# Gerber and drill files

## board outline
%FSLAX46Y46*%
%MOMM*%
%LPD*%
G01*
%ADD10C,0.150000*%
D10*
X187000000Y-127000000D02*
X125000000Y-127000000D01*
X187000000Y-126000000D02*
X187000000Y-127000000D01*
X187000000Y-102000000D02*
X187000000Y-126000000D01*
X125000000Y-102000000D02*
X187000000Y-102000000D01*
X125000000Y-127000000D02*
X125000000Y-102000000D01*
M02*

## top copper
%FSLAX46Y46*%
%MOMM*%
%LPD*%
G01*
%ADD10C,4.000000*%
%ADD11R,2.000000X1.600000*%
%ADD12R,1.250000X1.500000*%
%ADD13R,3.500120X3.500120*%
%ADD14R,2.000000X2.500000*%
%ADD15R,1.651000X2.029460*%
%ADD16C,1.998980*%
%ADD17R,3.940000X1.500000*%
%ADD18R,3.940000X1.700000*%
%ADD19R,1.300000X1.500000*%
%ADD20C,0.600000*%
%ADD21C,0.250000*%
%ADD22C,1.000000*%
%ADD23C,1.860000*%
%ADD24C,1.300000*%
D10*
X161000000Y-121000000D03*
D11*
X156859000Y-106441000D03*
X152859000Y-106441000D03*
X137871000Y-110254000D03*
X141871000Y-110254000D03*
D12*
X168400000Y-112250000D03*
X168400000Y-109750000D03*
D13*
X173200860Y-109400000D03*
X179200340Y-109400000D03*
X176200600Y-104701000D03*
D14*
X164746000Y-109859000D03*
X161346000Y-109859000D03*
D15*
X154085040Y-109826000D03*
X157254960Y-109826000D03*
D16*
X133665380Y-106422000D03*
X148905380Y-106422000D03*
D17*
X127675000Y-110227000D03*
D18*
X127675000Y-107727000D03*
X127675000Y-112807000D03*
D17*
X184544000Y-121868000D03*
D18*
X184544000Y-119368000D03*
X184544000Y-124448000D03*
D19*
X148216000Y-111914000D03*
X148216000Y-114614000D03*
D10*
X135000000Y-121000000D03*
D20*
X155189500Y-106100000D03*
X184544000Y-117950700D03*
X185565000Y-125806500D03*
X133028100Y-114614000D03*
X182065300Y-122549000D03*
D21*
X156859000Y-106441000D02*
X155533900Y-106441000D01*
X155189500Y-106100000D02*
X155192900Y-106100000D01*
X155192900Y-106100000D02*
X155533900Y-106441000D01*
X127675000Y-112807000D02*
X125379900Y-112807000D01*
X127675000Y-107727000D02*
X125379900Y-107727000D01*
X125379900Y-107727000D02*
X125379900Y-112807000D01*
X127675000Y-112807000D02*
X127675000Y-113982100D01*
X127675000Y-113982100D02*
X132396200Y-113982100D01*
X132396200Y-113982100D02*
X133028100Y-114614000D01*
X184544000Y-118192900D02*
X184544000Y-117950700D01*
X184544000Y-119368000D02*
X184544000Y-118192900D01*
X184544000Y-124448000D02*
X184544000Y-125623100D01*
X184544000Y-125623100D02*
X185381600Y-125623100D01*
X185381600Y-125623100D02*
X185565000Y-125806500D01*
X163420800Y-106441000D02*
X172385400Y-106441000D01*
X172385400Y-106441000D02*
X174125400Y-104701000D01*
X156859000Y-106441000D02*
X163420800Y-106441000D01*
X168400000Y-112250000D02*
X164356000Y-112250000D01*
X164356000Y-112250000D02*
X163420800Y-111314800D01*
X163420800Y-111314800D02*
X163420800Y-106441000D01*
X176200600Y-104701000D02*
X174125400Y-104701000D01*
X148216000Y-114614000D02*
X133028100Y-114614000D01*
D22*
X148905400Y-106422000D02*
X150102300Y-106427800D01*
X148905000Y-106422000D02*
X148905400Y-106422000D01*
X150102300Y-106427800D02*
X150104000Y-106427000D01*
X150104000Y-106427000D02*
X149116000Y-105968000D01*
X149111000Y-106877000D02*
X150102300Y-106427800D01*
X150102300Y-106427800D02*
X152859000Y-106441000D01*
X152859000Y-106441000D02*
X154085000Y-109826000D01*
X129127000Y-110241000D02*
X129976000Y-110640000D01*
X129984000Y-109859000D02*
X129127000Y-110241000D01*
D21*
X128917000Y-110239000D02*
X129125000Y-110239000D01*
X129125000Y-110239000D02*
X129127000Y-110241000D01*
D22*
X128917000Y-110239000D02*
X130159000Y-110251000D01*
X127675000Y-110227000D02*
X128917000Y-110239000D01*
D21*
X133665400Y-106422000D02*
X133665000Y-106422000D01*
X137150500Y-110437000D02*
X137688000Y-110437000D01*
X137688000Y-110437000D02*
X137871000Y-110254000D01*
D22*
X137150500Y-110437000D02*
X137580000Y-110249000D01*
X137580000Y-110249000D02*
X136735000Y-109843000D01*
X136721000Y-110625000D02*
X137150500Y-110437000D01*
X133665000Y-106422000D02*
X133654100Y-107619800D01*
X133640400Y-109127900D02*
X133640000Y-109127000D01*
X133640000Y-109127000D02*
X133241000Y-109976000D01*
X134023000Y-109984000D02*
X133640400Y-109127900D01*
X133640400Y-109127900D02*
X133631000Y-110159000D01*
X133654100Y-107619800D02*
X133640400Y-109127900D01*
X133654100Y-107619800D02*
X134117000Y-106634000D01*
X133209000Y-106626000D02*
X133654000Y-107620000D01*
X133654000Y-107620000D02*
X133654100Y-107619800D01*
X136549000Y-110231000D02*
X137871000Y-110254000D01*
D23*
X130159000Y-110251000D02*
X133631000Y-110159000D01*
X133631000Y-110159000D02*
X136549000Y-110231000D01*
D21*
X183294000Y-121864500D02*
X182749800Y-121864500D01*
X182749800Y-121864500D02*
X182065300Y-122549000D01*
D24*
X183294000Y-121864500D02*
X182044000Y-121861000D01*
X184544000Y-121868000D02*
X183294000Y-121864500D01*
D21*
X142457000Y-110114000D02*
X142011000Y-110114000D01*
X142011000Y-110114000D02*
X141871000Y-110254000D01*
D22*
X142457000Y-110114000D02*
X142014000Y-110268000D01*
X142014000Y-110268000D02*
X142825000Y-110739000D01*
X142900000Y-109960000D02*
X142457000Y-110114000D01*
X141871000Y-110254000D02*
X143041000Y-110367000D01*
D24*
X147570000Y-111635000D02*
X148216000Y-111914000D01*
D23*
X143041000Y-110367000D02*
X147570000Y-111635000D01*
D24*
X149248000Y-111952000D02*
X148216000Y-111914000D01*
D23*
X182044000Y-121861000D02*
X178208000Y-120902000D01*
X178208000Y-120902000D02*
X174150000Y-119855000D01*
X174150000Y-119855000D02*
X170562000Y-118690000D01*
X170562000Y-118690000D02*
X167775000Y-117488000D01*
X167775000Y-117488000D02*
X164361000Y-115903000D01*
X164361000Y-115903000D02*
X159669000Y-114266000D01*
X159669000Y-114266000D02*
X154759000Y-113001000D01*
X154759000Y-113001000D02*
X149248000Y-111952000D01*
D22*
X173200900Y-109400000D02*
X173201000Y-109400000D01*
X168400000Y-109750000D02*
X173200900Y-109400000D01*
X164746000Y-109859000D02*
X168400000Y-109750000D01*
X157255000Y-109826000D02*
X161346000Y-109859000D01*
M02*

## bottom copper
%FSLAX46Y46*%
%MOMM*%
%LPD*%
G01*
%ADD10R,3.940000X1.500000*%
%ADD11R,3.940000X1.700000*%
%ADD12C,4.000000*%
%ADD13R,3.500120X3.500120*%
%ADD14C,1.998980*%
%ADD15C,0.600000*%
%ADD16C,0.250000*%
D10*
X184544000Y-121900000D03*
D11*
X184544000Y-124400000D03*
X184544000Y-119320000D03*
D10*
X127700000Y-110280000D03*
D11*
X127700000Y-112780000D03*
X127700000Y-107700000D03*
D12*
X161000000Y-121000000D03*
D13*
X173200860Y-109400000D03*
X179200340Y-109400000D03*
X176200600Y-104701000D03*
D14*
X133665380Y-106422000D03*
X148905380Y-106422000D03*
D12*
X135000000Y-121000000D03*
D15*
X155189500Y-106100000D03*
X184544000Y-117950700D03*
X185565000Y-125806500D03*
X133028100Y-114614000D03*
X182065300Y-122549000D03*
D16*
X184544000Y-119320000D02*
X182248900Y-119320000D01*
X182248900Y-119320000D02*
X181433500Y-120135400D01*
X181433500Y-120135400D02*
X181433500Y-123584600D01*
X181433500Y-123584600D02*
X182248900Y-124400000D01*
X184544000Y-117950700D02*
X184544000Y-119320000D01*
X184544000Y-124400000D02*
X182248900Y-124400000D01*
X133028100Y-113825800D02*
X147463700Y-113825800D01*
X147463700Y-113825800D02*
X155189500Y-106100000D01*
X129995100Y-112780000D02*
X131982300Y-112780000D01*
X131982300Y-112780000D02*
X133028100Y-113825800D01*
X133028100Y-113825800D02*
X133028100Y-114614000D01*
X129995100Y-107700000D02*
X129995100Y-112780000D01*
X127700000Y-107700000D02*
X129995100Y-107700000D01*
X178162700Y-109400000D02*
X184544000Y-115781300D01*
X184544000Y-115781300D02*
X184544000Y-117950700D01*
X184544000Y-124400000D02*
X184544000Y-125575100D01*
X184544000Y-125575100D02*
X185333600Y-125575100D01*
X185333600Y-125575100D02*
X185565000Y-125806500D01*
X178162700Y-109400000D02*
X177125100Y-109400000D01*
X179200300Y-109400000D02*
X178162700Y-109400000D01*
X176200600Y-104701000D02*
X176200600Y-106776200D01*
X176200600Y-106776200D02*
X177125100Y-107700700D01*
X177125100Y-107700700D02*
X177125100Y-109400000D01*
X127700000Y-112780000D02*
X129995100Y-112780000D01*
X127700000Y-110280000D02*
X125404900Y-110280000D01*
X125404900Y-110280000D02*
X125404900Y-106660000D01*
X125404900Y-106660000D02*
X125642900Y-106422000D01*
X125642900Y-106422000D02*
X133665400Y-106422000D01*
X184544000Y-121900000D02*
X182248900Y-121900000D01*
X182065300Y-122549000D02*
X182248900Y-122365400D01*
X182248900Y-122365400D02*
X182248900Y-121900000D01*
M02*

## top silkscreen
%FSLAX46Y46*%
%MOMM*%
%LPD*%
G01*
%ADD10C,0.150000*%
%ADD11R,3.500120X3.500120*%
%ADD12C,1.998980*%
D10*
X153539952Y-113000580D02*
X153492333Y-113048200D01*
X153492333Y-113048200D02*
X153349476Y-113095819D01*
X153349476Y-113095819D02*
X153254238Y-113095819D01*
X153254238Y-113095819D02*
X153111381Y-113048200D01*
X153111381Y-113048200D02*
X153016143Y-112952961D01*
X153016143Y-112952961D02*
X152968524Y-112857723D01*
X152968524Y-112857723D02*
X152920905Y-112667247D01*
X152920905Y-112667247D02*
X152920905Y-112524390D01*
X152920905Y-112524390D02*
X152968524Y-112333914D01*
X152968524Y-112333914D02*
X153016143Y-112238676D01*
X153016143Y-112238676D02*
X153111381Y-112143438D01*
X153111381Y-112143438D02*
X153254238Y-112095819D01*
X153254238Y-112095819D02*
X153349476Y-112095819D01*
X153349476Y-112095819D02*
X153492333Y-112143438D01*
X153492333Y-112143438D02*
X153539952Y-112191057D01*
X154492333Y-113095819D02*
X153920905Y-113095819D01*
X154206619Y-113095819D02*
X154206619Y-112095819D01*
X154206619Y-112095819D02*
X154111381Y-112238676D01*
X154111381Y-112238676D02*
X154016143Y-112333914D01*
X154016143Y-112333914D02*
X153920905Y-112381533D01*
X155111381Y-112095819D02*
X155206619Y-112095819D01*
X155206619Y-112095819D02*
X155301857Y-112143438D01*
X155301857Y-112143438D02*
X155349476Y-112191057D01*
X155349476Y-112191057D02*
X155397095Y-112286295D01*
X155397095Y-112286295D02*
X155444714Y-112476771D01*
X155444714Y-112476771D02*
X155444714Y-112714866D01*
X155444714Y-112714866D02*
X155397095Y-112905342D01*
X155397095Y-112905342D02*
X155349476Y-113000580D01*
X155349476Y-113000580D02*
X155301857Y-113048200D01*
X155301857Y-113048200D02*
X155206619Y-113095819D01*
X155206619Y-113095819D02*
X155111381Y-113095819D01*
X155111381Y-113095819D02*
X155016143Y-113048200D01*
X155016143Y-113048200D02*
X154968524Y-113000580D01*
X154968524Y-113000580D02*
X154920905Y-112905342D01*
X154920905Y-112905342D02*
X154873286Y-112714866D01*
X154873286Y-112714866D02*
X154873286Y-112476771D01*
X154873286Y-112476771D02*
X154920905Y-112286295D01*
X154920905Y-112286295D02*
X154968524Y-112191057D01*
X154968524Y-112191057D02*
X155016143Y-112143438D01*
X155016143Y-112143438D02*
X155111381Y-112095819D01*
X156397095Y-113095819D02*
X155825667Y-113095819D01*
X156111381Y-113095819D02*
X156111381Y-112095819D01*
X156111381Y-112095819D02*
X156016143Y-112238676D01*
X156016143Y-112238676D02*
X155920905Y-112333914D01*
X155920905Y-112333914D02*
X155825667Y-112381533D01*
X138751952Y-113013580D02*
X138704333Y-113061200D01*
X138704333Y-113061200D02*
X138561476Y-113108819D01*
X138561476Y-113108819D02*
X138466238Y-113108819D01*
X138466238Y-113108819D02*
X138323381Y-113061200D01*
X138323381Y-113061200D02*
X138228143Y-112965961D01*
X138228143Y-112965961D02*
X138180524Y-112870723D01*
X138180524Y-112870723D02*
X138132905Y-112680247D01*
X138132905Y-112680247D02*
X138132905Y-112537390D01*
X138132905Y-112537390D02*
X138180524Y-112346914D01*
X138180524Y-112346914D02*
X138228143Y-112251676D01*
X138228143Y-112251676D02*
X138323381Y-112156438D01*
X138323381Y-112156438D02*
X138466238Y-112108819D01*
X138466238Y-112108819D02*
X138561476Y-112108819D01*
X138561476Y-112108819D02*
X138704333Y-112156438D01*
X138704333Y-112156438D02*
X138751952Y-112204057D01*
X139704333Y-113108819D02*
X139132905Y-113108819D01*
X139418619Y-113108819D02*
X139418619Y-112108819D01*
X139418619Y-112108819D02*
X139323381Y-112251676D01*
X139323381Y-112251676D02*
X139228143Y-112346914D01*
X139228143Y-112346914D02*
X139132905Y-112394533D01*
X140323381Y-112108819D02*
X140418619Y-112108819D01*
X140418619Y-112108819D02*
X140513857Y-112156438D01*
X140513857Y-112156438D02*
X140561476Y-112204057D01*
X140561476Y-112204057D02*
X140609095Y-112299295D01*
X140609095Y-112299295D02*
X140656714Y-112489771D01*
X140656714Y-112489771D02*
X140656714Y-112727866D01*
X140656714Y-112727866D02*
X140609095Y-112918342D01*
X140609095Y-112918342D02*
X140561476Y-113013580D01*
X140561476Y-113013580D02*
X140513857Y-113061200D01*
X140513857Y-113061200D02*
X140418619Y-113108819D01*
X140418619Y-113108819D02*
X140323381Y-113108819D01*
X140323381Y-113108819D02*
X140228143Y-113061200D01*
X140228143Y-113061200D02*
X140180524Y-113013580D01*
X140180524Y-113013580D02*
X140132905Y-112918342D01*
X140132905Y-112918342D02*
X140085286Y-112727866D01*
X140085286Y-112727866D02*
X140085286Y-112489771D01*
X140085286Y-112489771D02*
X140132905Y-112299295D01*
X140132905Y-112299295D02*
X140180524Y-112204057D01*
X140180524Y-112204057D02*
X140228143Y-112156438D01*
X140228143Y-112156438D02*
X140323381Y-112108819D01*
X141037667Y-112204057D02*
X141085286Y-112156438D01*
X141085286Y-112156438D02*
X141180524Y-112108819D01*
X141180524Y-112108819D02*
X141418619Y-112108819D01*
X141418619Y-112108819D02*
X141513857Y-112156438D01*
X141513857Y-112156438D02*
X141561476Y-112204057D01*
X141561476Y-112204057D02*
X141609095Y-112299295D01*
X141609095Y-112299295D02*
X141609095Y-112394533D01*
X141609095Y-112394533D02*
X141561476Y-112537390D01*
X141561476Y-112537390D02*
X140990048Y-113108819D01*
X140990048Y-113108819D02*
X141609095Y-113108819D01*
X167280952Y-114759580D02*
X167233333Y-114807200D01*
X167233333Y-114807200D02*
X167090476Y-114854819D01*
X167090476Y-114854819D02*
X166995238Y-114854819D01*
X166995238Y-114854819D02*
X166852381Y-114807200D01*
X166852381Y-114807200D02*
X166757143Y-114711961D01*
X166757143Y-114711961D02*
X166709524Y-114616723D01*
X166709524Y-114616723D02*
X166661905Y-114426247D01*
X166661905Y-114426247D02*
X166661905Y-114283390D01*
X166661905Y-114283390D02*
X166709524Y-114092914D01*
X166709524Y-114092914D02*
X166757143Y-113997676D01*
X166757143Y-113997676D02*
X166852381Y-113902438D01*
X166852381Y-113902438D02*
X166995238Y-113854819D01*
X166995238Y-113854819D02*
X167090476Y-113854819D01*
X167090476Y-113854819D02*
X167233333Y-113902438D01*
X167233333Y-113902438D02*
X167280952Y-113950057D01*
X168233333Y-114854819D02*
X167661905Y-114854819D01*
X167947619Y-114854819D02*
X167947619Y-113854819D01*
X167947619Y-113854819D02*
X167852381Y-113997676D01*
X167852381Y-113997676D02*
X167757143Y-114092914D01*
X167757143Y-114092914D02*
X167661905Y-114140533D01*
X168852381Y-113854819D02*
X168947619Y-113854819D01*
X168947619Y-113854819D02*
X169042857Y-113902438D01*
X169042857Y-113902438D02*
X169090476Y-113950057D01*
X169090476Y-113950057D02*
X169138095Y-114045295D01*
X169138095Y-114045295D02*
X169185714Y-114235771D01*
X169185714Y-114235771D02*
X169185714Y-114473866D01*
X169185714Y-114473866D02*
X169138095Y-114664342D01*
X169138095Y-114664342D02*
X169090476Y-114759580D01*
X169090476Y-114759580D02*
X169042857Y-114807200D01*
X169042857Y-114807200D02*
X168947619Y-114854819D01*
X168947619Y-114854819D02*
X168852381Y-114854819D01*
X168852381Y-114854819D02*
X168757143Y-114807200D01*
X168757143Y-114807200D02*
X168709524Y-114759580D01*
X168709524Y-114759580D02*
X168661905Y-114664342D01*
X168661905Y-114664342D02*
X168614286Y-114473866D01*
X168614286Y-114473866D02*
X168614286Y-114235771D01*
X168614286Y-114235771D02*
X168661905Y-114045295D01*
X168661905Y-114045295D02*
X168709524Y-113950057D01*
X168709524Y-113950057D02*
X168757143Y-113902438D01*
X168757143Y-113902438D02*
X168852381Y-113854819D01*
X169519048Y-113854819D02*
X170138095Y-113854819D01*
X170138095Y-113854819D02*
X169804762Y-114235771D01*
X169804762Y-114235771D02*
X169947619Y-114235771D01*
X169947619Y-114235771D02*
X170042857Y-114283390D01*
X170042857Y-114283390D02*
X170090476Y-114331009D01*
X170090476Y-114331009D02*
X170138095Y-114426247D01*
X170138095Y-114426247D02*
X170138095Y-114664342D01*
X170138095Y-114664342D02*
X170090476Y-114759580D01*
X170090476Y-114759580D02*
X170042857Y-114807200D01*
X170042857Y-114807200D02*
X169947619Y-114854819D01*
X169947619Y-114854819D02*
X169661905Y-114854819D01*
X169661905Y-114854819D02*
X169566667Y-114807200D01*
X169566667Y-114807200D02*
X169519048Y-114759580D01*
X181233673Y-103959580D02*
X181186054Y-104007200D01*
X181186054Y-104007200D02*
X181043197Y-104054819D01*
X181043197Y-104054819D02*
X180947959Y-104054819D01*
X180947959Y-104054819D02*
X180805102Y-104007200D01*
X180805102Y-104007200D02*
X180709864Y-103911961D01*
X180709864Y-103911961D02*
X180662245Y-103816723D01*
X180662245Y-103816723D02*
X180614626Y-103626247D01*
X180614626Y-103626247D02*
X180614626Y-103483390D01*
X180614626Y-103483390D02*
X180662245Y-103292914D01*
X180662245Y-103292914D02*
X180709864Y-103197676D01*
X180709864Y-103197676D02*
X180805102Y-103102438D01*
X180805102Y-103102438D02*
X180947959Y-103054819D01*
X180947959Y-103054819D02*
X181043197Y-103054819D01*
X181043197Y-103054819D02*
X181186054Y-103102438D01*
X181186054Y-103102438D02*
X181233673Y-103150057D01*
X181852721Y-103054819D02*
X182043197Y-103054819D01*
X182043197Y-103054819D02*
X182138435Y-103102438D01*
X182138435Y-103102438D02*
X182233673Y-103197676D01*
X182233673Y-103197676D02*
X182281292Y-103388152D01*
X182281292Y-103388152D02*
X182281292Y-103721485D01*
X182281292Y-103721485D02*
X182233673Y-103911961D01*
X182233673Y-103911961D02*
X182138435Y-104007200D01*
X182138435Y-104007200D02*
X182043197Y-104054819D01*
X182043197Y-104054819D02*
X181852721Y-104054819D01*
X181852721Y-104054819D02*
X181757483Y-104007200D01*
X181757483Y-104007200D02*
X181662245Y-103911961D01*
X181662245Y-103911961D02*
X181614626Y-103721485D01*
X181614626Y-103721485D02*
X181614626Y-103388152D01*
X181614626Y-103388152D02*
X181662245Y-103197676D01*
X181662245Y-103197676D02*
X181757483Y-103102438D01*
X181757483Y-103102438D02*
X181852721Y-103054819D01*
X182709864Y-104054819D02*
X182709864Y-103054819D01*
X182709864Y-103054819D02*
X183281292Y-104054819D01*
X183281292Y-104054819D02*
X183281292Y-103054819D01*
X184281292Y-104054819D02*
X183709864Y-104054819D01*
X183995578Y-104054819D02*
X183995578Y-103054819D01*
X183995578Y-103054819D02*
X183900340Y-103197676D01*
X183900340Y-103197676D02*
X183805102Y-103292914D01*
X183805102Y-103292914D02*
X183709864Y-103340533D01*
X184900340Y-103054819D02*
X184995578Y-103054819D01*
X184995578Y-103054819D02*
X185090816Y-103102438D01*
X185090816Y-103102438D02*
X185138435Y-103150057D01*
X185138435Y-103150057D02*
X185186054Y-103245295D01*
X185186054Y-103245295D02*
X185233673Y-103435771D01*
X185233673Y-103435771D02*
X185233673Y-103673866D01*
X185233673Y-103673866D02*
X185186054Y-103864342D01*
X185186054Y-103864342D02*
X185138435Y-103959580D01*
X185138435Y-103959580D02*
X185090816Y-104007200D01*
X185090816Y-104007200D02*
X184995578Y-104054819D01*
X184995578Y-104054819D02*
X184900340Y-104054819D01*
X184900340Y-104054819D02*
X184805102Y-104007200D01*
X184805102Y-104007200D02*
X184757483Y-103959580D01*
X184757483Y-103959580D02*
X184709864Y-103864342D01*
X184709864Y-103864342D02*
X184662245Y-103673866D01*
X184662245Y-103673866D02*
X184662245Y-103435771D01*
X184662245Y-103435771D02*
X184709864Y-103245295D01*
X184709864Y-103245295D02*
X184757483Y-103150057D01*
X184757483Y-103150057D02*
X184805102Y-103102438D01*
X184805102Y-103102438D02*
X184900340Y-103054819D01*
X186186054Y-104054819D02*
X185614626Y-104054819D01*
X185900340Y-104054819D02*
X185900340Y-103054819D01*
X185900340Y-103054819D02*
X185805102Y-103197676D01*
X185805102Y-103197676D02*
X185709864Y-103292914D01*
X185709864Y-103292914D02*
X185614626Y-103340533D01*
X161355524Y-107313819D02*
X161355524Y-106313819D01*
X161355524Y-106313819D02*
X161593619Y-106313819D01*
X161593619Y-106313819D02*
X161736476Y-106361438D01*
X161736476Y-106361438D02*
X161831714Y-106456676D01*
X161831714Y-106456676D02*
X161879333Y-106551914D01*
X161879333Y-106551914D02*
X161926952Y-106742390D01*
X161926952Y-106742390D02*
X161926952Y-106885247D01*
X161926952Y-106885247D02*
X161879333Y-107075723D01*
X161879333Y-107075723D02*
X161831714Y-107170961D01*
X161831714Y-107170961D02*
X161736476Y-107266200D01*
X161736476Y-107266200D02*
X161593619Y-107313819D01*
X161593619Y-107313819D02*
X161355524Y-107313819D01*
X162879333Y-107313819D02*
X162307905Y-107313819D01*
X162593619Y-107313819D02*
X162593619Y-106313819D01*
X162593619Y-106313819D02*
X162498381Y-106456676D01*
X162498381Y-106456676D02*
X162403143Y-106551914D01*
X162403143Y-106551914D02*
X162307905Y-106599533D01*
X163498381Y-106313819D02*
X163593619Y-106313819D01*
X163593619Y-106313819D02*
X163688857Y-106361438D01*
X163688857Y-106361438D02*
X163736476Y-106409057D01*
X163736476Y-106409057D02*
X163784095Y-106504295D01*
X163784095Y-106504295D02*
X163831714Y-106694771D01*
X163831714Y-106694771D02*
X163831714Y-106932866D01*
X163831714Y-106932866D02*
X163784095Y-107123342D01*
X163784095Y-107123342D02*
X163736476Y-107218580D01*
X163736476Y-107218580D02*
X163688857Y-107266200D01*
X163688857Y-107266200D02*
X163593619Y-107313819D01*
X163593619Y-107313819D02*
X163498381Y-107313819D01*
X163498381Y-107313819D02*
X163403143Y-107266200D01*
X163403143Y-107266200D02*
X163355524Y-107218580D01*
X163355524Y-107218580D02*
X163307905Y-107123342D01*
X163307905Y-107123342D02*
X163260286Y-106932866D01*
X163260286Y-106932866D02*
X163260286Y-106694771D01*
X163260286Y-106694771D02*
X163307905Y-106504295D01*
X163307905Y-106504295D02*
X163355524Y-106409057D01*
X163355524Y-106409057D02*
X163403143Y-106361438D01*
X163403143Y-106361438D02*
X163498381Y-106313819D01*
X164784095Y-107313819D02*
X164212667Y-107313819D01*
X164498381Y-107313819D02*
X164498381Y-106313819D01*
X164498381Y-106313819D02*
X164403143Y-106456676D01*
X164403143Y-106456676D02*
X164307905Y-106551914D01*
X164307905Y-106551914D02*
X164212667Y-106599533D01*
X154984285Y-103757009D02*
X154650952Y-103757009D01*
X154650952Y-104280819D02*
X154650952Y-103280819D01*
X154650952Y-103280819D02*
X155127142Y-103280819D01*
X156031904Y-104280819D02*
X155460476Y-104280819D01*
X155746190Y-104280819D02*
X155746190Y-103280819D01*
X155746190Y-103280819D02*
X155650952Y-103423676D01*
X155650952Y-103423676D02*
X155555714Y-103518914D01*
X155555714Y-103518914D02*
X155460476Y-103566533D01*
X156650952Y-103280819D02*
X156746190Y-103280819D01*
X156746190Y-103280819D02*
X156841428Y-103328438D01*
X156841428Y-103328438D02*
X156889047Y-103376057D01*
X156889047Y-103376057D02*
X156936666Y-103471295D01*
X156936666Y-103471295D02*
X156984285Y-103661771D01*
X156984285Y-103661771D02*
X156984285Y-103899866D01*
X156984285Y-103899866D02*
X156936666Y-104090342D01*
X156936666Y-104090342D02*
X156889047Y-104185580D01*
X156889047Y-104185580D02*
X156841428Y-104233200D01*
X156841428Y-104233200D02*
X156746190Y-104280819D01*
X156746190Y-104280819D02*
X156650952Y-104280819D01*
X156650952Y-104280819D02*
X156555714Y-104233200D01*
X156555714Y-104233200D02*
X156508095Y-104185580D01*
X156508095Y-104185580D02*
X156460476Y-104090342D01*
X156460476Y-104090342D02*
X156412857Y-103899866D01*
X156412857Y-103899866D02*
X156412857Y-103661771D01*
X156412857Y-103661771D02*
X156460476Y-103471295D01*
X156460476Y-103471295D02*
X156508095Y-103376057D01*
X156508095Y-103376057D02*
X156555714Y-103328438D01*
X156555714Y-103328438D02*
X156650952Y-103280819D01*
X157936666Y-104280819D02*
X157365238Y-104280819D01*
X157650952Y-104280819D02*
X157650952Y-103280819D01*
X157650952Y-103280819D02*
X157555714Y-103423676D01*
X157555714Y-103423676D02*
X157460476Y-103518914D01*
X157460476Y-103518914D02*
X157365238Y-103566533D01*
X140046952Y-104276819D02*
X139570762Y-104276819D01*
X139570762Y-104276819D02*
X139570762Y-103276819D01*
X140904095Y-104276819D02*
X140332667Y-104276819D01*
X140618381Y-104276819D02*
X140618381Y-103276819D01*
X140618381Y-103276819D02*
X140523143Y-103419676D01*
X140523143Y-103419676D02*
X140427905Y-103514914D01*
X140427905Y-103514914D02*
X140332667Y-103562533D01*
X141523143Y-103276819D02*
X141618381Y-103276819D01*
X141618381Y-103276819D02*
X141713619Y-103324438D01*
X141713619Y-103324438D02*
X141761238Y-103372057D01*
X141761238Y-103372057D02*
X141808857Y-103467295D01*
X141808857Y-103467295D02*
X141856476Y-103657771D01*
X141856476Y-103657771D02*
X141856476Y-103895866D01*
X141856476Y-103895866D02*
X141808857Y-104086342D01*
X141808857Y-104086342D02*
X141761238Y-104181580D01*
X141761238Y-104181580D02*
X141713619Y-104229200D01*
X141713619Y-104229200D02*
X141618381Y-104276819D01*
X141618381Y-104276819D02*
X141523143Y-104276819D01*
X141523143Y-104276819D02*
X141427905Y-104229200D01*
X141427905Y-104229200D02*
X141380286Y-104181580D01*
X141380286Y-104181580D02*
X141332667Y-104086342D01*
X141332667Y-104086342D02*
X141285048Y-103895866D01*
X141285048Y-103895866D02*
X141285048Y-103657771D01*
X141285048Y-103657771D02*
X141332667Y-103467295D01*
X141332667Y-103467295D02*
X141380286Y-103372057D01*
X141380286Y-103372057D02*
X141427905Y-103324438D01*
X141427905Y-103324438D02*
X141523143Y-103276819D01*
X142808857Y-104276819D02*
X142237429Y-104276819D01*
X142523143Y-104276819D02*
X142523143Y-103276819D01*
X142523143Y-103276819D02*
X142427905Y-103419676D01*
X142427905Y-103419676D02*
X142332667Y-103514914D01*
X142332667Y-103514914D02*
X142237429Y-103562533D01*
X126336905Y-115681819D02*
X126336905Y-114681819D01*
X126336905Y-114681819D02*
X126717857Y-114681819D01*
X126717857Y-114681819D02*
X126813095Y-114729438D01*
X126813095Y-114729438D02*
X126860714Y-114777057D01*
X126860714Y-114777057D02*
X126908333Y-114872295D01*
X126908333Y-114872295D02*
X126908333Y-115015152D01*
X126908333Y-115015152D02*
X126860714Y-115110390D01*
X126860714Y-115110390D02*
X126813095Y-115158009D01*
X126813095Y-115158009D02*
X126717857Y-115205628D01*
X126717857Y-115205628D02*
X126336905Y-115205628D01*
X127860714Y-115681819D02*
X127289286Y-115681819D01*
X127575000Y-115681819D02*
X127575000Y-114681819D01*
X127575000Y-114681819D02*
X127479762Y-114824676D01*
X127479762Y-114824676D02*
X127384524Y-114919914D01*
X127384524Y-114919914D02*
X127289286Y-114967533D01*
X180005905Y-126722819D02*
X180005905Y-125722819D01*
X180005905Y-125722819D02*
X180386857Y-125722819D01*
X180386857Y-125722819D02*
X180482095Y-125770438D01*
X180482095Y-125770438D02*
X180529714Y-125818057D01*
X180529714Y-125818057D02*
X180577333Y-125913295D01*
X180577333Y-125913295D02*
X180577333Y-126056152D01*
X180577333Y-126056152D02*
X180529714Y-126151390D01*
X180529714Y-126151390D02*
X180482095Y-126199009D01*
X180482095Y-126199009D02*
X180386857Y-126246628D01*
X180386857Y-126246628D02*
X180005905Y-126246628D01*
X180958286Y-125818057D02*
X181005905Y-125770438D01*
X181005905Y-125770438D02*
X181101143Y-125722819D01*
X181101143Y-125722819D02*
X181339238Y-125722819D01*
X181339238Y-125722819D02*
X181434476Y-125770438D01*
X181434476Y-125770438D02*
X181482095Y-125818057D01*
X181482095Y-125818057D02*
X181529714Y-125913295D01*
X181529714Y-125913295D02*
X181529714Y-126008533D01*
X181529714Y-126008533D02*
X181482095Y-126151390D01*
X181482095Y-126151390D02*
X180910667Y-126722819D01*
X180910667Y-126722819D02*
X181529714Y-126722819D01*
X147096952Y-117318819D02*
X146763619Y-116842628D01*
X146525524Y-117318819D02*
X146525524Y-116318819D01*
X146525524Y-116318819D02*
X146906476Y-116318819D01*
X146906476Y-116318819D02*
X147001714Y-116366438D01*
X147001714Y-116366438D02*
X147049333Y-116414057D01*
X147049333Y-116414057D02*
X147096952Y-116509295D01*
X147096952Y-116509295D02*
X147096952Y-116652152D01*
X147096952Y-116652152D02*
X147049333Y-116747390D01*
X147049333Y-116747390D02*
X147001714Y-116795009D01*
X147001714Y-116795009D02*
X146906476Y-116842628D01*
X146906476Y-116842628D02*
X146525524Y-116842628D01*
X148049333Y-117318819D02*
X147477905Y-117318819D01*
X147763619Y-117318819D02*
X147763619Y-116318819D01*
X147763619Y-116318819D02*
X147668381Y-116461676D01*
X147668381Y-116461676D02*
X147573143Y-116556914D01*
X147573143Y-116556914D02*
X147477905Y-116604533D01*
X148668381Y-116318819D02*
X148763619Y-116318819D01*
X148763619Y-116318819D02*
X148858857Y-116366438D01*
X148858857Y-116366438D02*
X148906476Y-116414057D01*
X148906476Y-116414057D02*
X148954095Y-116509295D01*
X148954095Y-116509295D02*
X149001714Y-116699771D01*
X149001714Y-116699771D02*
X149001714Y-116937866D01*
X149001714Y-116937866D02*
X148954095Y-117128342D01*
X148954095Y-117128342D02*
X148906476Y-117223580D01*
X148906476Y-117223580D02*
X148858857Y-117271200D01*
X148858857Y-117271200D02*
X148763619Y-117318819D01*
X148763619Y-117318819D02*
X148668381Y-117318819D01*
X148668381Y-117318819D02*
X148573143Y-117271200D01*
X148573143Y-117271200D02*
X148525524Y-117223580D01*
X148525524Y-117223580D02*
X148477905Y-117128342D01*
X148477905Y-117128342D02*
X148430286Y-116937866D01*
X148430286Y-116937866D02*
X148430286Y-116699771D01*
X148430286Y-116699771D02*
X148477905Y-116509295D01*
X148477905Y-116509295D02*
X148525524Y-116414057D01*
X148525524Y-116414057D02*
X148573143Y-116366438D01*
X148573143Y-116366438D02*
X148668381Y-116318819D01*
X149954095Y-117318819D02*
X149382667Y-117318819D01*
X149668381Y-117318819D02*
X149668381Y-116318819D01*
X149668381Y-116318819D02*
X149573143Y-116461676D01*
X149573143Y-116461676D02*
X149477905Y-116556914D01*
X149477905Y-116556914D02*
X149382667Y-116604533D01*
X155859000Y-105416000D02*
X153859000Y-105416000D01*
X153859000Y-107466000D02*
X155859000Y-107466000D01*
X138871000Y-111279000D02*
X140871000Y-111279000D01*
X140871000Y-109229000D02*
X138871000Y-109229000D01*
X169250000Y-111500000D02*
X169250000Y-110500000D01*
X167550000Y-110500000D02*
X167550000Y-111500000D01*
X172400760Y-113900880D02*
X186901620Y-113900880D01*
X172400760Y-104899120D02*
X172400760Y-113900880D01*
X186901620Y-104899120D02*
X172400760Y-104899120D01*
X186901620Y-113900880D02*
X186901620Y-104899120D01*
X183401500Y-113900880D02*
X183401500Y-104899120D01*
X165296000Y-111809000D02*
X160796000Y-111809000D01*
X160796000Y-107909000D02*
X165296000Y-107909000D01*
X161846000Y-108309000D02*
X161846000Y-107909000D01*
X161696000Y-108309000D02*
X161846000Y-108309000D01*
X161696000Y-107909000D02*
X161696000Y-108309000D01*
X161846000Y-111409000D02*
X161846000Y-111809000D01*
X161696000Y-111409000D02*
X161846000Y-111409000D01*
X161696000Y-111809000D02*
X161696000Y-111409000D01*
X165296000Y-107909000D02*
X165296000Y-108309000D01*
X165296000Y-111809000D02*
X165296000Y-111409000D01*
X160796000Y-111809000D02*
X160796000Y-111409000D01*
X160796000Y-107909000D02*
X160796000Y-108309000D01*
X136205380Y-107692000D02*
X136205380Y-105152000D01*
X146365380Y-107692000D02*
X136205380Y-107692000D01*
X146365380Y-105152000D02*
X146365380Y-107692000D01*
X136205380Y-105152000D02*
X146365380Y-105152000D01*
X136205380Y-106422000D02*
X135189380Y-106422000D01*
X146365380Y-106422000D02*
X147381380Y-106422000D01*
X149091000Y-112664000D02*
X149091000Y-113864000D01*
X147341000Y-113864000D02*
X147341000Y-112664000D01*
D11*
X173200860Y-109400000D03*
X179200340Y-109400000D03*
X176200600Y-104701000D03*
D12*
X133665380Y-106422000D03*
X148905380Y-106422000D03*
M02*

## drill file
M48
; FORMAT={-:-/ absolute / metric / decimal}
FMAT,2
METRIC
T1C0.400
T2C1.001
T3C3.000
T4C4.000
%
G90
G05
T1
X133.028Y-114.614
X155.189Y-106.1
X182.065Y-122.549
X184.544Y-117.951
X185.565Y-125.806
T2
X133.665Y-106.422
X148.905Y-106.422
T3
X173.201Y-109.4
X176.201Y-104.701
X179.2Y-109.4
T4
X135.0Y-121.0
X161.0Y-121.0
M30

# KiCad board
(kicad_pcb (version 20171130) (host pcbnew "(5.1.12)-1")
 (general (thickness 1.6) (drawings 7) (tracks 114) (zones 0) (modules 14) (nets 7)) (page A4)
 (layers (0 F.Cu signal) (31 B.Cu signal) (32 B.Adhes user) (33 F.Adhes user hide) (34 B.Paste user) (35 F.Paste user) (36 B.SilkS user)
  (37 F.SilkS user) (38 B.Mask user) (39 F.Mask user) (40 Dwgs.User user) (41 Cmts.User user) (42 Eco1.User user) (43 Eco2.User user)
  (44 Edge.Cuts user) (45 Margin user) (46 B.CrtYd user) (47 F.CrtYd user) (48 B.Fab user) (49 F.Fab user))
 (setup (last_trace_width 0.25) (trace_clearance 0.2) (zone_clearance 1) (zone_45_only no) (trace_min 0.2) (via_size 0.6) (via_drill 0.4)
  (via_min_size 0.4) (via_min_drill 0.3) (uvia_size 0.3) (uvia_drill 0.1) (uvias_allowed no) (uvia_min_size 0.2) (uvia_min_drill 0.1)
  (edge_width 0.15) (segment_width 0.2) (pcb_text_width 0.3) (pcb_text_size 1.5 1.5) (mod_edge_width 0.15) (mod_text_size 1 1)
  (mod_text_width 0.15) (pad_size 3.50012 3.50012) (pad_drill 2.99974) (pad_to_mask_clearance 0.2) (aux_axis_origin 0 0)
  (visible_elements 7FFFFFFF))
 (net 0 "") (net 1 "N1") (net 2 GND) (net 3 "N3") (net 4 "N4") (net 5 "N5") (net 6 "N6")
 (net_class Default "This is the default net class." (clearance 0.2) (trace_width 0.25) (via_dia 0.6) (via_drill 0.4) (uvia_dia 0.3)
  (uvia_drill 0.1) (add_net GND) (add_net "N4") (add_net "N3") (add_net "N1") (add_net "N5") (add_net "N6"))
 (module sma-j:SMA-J (layer B.Cu) (at 184.544 124.4)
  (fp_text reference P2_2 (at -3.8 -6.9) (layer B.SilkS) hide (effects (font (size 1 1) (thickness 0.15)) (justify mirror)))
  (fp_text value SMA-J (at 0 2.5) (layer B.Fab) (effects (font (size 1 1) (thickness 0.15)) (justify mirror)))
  (pad 1 smd rect (at 0 -2.5) (size 3.94 1.5) (layers B.Cu B.Paste B.Mask) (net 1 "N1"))
  (pad 2 smd rect (at 0 0) (size 3.94 1.7) (layers B.Cu B.Paste B.Mask) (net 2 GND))
  (pad 2 smd rect (at 0 -5.08) (size 3.94 1.7) (layers B.Cu B.Paste B.Mask) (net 2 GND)))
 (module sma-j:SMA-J (layer B.Cu) (at 127.7 112.78)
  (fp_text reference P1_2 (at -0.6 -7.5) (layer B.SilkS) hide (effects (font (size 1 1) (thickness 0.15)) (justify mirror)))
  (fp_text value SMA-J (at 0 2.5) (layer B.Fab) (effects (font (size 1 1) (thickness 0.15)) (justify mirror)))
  (pad 1 smd rect (at 0 -2.5) (size 3.94 1.5) (layers B.Cu B.Paste B.Mask) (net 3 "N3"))
  (pad 2 smd rect (at 0 0) (size 3.94 1.7) (layers B.Cu B.Paste B.Mask) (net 2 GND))
  (pad 2 smd rect (at 0 -5.08) (size 3.94 1.7) (layers B.Cu B.Paste B.Mask) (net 2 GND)))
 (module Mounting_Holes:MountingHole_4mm (layer F.Cu) (at 161 121)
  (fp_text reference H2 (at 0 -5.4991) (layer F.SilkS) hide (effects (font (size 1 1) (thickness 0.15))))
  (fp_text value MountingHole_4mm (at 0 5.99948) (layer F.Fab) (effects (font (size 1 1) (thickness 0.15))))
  (pad 1 thru_hole circle (at 0 0) (size 4 4) (drill 4) (layers *.Cu *.Mask)))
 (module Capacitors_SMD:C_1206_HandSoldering (layer F.Cu) (at 154.859 106.441 180)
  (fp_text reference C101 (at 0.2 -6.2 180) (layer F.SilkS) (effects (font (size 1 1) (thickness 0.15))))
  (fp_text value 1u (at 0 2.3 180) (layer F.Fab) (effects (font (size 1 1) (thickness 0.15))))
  (fp_line (start -1 1.025) (end 1 1.025) (layer F.SilkS) (width 0.15))
  (fp_line (start 1 -1.025) (end -1 -1.025) (layer F.SilkS) (width 0.15))
  (pad 1 smd rect (at -2 0 180) (size 2 1.6) (layers F.Cu F.Paste F.Mask) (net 2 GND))
  (pad 2 smd rect (at 2 0 180) (size 2 1.6) (layers F.Cu F.Paste F.Mask) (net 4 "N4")))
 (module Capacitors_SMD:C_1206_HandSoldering (layer F.Cu) (at 139.871 110.254)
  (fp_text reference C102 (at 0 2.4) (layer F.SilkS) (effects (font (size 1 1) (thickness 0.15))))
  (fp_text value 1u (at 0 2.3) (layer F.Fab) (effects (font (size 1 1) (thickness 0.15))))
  (fp_line (start -1 1.025) (end 1 1.025) (layer F.SilkS) (width 0.15))
  (fp_line (start 1 -1.025) (end -1 -1.025) (layer F.SilkS) (width 0.15))
  (pad 1 smd rect (at -2 0) (size 2 1.6) (layers F.Cu F.Paste F.Mask) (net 3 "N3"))
  (pad 2 smd rect (at 2 0) (size 2 1.6) (layers F.Cu F.Paste F.Mask) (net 1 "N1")))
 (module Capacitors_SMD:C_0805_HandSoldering (layer F.Cu) (at 168.4 111 90)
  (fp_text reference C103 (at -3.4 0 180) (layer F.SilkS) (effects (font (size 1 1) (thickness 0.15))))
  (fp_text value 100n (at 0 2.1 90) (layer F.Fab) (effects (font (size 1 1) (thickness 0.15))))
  (fp_line (start -0.5 0.85) (end 0.5 0.85) (layer F.SilkS) (width 0.15))
  (fp_line (start 0.5 -0.85) (end -0.5 -0.85) (layer F.SilkS) (width 0.15))
  (pad 1 smd rect (at -1.25 0 90) (size 1.5 1.25) (layers F.Cu F.Paste F.Mask) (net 2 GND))
  (pad 2 smd rect (at 1.25 0 90) (size 1.5 1.25) (layers F.Cu F.Paste F.Mask) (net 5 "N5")))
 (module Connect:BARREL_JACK (layer F.Cu) (at 179.401 109.4 180)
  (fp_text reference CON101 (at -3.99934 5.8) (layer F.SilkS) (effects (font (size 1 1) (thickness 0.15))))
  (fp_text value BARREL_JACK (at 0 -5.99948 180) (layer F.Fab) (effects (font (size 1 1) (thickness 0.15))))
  (fp_line (start 7.00024 -4.50088) (end -7.50062 -4.50088) (layer F.SilkS) (width 0.15))
  (fp_line (start 7.00024 4.50088) (end 7.00024 -4.50088) (layer F.SilkS) (width 0.15))
  (fp_line (start -7.50062 4.50088) (end 7.00024 4.50088) (layer F.SilkS) (width 0.15))
  (fp_line (start -7.50062 -4.50088) (end -7.50062 4.50088) (layer F.SilkS) (width 0.15))
  (fp_line (start -4.0005 -4.50088) (end -4.0005 4.50088) (layer F.SilkS) (width 0.15))
  (pad 1 thru_hole rect (at 6.20014 0 180) (size 3.50012 3.50012) (drill 2.99974) (layers *.Cu *.Mask F.SilkS) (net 5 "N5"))
  (pad 2 thru_hole rect (at 0.20066 0 180) (size 3.50012 3.50012) (drill 2.99974) (layers *.Cu *.Mask F.SilkS) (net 2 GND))
  (pad 3 thru_hole rect (at 3.2004 4.699 180) (size 3.50012 3.50012) (drill 2.99974) (layers *.Cu *.Mask F.SilkS) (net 2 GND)))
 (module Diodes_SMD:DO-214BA (layer F.Cu) (at 163.046 109.859)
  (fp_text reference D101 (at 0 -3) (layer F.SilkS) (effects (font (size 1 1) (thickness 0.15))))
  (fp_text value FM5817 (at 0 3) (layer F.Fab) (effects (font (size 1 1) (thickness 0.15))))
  (fp_line (start 2.25 1.95) (end -2.25 1.95) (layer F.SilkS) (width 0.15))
  (fp_line (start -2.25 -1.95) (end 2.25 -1.95) (layer F.SilkS) (width 0.15))
  (fp_line (start -1.2 -1.55) (end -1.2 -1.95) (layer F.SilkS) (width 0.15))
  (fp_line (start -1.35 -1.55) (end -1.2 -1.55) (layer F.SilkS) (width 0.15))
  (fp_line (start -1.35 -1.95) (end -1.35 -1.55) (layer F.SilkS) (width 0.15))
  (fp_line (start -1.2 1.55) (end -1.2 1.95) (layer F.SilkS) (width 0.15))
  (fp_line (start -1.35 1.55) (end -1.2 1.55) (layer F.SilkS) (width 0.15))
  (fp_line (start -1.35 1.95) (end -1.35 1.55) (layer F.SilkS) (width 0.15))
  (fp_line (start 2.25 -1.95) (end 2.25 -1.55) (layer F.SilkS) (width 0.15))
  (fp_line (start 2.25 1.95) (end 2.25 1.55) (layer F.SilkS) (width 0.15))
  (fp_line (start -2.25 1.95) (end -2.25 1.55) (layer F.SilkS) (width 0.15))
  (fp_line (start -2.25 -1.95) (end -2.25 -1.55) (layer F.SilkS) (width 0.15))
  (pad 2 smd rect (at 1.7 0) (size 2 2.5) (layers F.Cu F.Paste F.Mask) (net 5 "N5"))
  (pad 1 smd rect (at -1.7 0) (size 2 2.5) (layers F.Cu F.Paste F.Mask) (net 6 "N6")))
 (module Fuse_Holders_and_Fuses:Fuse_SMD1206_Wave (layer F.Cu) (at 155.67 109.826)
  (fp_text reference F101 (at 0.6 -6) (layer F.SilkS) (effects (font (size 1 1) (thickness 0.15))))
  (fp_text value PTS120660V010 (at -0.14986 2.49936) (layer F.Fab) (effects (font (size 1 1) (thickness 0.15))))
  (pad 1 smd rect (at -1.58496 0 90) (size 2.02946 1.651) (layers F.Cu F.Paste F.Mask) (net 4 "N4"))
  (pad 2 smd rect (at 1.58496 0 90) (size 2.02946 1.651) (layers F.Cu F.Paste F.Mask) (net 6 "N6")))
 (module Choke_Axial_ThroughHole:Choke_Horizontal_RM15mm (layer F.Cu) (at 141.166 106.422)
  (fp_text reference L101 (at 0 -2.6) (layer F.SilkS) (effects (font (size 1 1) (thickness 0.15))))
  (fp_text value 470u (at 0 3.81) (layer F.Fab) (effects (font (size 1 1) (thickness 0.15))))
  (fp_line (start -4.96062 1.27) (end -4.96062 -1.27) (layer F.SilkS) (width 0.15))
  (fp_line (start 5.19938 1.27) (end -4.96062 1.27) (layer F.SilkS) (width 0.15))
  (fp_line (start 5.19938 -1.27) (end 5.19938 1.27) (layer F.SilkS) (width 0.15))
  (fp_line (start -4.96062 -1.27) (end 5.19938 -1.27) (layer F.SilkS) (width 0.15))
  (fp_line (start -4.96062 0) (end -5.97662 0) (layer F.SilkS) (width 0.15))
  (fp_line (start 5.19938 0) (end 6.21538 0) (layer F.SilkS) (width 0.15))
  (pad 1 thru_hole circle (at -7.50062 0) (size 1.99898 1.99898) (drill 1.00076) (layers *.Cu *.Mask F.SilkS) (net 3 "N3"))
  (pad 2 thru_hole circle (at 7.73938 0) (size 1.99898 1.99898) (drill 1.00076) (layers *.Cu *.Mask F.SilkS) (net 4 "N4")))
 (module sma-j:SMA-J (layer F.Cu) (at 127.675 107.727)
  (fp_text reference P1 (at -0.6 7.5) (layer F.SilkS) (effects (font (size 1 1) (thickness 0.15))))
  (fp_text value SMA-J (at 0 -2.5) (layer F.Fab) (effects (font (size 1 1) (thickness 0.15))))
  (pad 1 smd rect (at 0 2.5) (size 3.94 1.5) (layers F.Cu F.Paste F.Mask) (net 3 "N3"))
  (pad 2 smd rect (at 0 0) (size 3.94 1.7) (layers F.Cu F.Paste F.Mask) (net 2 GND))
  (pad 2 smd rect (at 0 5.08) (size 3.94 1.7) (layers F.Cu F.Paste F.Mask) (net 2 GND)))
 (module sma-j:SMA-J (layer F.Cu) (at 184.544 119.368)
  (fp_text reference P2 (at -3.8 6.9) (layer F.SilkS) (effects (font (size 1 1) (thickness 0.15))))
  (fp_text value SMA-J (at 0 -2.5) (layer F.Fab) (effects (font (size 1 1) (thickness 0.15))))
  (pad 1 smd rect (at 0 2.5) (size 3.94 1.5) (layers F.Cu F.Paste F.Mask) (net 1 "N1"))
  (pad 2 smd rect (at 0 0) (size 3.94 1.7) (layers F.Cu F.Paste F.Mask) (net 2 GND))
  (pad 2 smd rect (at 0 5.08) (size 3.94 1.7) (layers F.Cu F.Paste F.Mask) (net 2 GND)))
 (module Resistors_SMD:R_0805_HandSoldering (layer F.Cu) (at 148.216 113.264 270)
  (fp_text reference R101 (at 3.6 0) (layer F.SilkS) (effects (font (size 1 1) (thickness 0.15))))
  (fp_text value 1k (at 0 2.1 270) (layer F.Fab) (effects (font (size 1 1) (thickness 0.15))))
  (fp_line (start -0.6 -0.875) (end 0.6 -0.875) (layer F.SilkS) (width 0.15))
  (fp_line (start 0.6 0.875) (end -0.6 0.875) (layer F.SilkS) (width 0.15))
  (pad 1 smd rect (at -1.35 0 270) (size 1.5 1.3) (layers F.Cu F.Paste F.Mask) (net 1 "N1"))
  (pad 2 smd rect (at 1.35 0 270) (size 1.5 1.3) (layers F.Cu F.Paste F.Mask) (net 2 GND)))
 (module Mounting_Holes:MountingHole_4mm (layer F.Cu) (at 135 121)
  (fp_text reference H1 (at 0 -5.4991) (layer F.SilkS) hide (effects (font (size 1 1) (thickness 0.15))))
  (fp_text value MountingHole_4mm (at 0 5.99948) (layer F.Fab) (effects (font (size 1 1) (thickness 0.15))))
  (pad 1 thru_hole circle (at 0 0) (size 4 4) (drill 4) (layers *.Cu *.Mask)))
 (gr_line (start 187 127) (end 125 127) (layer Edge.Cuts) (width 0.15))
 (gr_line (start 187 126) (end 187 127) (layer Edge.Cuts) (width 0.15))
 (gr_line (start 187 102) (end 187 126) (layer Edge.Cuts) (width 0.15))
 (gr_line (start 125 102) (end 187 102) (layer Edge.Cuts) (width 0.15))
 (gr_line (start 125 127) (end 125 102) (layer Edge.Cuts) (width 0.15))
 (segment (start 184.544 119.32) (end 182.2489 119.32) (width 0.25) (layer B.Cu) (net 2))
 (segment (start 182.2489 119.32) (end 181.4335 120.1354) (width 0.25) (layer B.Cu) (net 2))
 (segment (start 181.4335 120.1354) (end 181.4335 123.5846) (width 0.25) (layer B.Cu) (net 2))
 (segment (start 181.4335 123.5846) (end 182.2489 124.4) (width 0.25) (layer B.Cu) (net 2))
 (segment (start 184.544 117.9507) (end 184.544 119.32) (width 0.25) (layer B.Cu) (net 2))
 (segment (start 184.544 124.4) (end 182.2489 124.4) (width 0.25) (layer B.Cu) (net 2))
 (segment (start 133.0281 113.8258) (end 147.4637 113.8258) (width 0.25) (layer B.Cu) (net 2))
 (segment (start 147.4637 113.8258) (end 155.1895 106.1) (width 0.25) (layer B.Cu) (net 2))
 (segment (start 129.9951 112.78) (end 131.9823 112.78) (width 0.25) (layer B.Cu) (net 2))
 (segment (start 131.9823 112.78) (end 133.0281 113.8258) (width 0.25) (layer B.Cu) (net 2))
 (segment (start 133.0281 113.8258) (end 133.0281 114.614) (width 0.25) (layer B.Cu) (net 2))
 (segment (start 156.859 106.441) (end 155.5339 106.441) (width 0.25) (layer F.Cu) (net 2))
 (segment (start 155.1895 106.1) (end 155.1929 106.1) (width 0.25) (layer F.Cu) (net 2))
 (segment (start 155.1929 106.1) (end 155.5339 106.441) (width 0.25) (layer F.Cu) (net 2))
 (segment (start 129.9951 107.7) (end 129.9951 112.78) (width 0.25) (layer B.Cu) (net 2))
 (segment (start 127.7 107.7) (end 129.9951 107.7) (width 0.25) (layer B.Cu) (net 2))
 (segment (start 127.675 112.807) (end 125.3799 112.807) (width 0.25) (layer F.Cu) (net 2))
 (segment (start 127.675 107.727) (end 125.3799 107.727) (width 0.25) (layer F.Cu) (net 2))
 (segment (start 125.3799 107.727) (end 125.3799 112.807) (width 0.25) (layer F.Cu) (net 2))
 (segment (start 127.675 112.807) (end 127.675 113.9821) (width 0.25) (layer F.Cu) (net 2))
 (segment (start 127.675 113.9821) (end 132.3962 113.9821) (width 0.25) (layer F.Cu) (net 2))
 (segment (start 132.3962 113.9821) (end 133.0281 114.614) (width 0.25) (layer F.Cu) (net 2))
 (segment (start 184.544 118.1929) (end 184.544 117.9507) (width 0.25) (layer F.Cu) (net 2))
 (segment (start 178.1627 109.4) (end 184.544 115.7813) (width 0.25) (layer B.Cu) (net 2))
 (segment (start 184.544 115.7813) (end 184.544 117.9507) (width 0.25) (layer B.Cu) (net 2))
 (segment (start 184.544 119.368) (end 184.544 118.1929) (width 0.25) (layer F.Cu) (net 2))
 (segment (start 184.544 124.4) (end 184.544 125.5751) (width 0.25) (layer B.Cu) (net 2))
 (segment (start 184.544 124.448) (end 184.544 125.6231) (width 0.25) (layer F.Cu) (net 2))
 (segment (start 184.544 125.6231) (end 185.3816 125.6231) (width 0.25) (layer F.Cu) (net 2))
 (segment (start 185.3816 125.6231) (end 185.565 125.8065) (width 0.25) (layer F.Cu) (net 2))
 (segment (start 184.544 125.5751) (end 185.3336 125.5751) (width 0.25) (layer B.Cu) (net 2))
 (segment (start 185.3336 125.5751) (end 185.565 125.8065) (width 0.25) (layer B.Cu) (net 2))
 (segment (start 163.4208 106.441) (end 172.3854 106.441) (width 0.25) (layer F.Cu) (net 2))
 (segment (start 172.3854 106.441) (end 174.1254 104.701) (width 0.25) (layer F.Cu) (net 2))
 (segment (start 156.859 106.441) (end 163.4208 106.441) (width 0.25) (layer F.Cu) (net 2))
 (segment (start 168.4 112.25) (end 164.356 112.25) (width 0.25) (layer F.Cu) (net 2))
 (segment (start 164.356 112.25) (end 163.4208 111.3148) (width 0.25) (layer F.Cu) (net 2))
 (segment (start 163.4208 111.3148) (end 163.4208 106.441) (width 0.25) (layer F.Cu) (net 2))
 (segment (start 176.2006 104.701) (end 174.1254 104.701) (width 0.25) (layer F.Cu) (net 2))
 (segment (start 178.1627 109.4) (end 177.1251 109.4) (width 0.25) (layer B.Cu) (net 2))
 (segment (start 179.2003 109.4) (end 178.1627 109.4) (width 0.25) (layer B.Cu) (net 2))
 (segment (start 176.2006 104.701) (end 176.2006 106.7762) (width 0.25) (layer B.Cu) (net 2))
 (segment (start 176.2006 106.7762) (end 177.1251 107.7007) (width 0.25) (layer B.Cu) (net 2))
 (segment (start 177.1251 107.7007) (end 177.1251 109.4) (width 0.25) (layer B.Cu) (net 2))
 (segment (start 148.216 114.614) (end 133.0281 114.614) (width 0.25) (layer F.Cu) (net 2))
 (segment (start 127.7 112.78) (end 129.9951 112.78) (width 0.25) (layer B.Cu) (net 2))
 (via (at 155.1895 106.1) (size 0.6) (layers F.Cu B.Cu) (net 2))
 (via (at 184.544 117.9507) (size 0.6) (layers F.Cu B.Cu) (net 2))
 (via (at 185.565 125.8065) (size 0.6) (layers F.Cu B.Cu) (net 2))
 (via (at 133.0281 114.614) (size 0.6) (layers F.Cu B.Cu) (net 2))
 (segment (start 148.9054 106.422) (end 150.1023 106.4278) (width 1) (layer F.Cu) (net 4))
 (segment (start 148.905 106.422) (end 148.9054 106.422) (width 1) (layer F.Cu) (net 4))
 (segment (start 150.1023 106.4278) (end 150.104 106.427) (width 1) (layer F.Cu) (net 4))
 (segment (start 150.104 106.427) (end 149.116 105.968) (width 1) (layer F.Cu) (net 4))
 (segment (start 149.111 106.877) (end 150.1023 106.4278) (width 1) (layer F.Cu) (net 4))
 (segment (start 150.1023 106.4278) (end 152.859 106.441) (width 1) (layer F.Cu) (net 4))
 (segment (start 152.859 106.441) (end 154.085 109.826) (width 1) (layer F.Cu) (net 4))
 (segment (start 129.127 110.241) (end 129.976 110.64) (width 1) (layer F.Cu) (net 3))
 (segment (start 129.984 109.859) (end 129.127 110.241) (width 1) (layer F.Cu) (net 3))
 (segment (start 128.917 110.239) (end 129.125 110.239) (width 0.25) (layer F.Cu) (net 3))
 (segment (start 129.125 110.239) (end 129.127 110.241) (width 0.25) (layer F.Cu) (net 3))
 (segment (start 128.917 110.239) (end 130.159 110.251) (width 1) (layer F.Cu) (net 3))
 (segment (start 127.675 110.227) (end 128.917 110.239) (width 1) (layer F.Cu) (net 3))
 (segment (start 127.7 110.28) (end 125.4049 110.28) (width 0.25) (layer B.Cu) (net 3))
 (segment (start 125.4049 110.28) (end 125.4049 106.66) (width 0.25) (layer B.Cu) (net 3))
 (segment (start 125.4049 106.66) (end 125.6429 106.422) (width 0.25) (layer B.Cu) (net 3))
 (segment (start 125.6429 106.422) (end 133.6654 106.422) (width 0.25) (layer B.Cu) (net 3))
 (segment (start 133.6654 106.422) (end 133.665 106.422) (width 0.25) (layer F.Cu) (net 3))
 (segment (start 137.1505 110.437) (end 137.688 110.437) (width 0.25) (layer F.Cu) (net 3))
 (segment (start 137.688 110.437) (end 137.871 110.254) (width 0.25) (layer F.Cu) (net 3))
 (segment (start 137.1505 110.437) (end 137.58 110.249) (width 1) (layer F.Cu) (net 3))
 (segment (start 137.58 110.249) (end 136.735 109.843) (width 1) (layer F.Cu) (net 3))
 (segment (start 136.721 110.625) (end 137.1505 110.437) (width 1) (layer F.Cu) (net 3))
 (segment (start 133.665 106.422) (end 133.6541 107.6198) (width 1) (layer F.Cu) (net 3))
 (segment (start 133.6404 109.1279) (end 133.64 109.127) (width 1) (layer F.Cu) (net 3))
 (segment (start 133.64 109.127) (end 133.241 109.976) (width 1) (layer F.Cu) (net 3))
 (segment (start 134.023 109.984) (end 133.6404 109.1279) (width 1) (layer F.Cu) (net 3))
 (segment (start 133.6404 109.1279) (end 133.631 110.159) (width 1) (layer F.Cu) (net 3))
 (segment (start 133.6541 107.6198) (end 133.6404 109.1279) (width 1) (layer F.Cu) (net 3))
 (segment (start 133.6541 107.6198) (end 134.117 106.634) (width 1) (layer F.Cu) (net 3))
 (segment (start 133.209 106.626) (end 133.654 107.62) (width 1) (layer F.Cu) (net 3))
 (segment (start 133.654 107.62) (end 133.6541 107.6198) (width 1) (layer F.Cu) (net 3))
 (segment (start 136.549 110.231) (end 137.871 110.254) (width 1) (layer F.Cu) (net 3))
 (segment (start 130.159 110.251) (end 133.631 110.159) (width 1.86) (layer F.Cu) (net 3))
 (segment (start 133.631 110.159) (end 136.549 110.231) (width 1.86) (layer F.Cu) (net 3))
 (segment (start 184.544 121.9) (end 182.2489 121.9) (width 0.25) (layer B.Cu) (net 1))
 (segment (start 183.294 121.8645) (end 182.7498 121.8645) (width 0.25) (layer F.Cu) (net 1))
 (segment (start 182.7498 121.8645) (end 182.0653 122.549) (width 0.25) (layer F.Cu) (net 1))
 (segment (start 182.0653 122.549) (end 182.2489 122.3654) (width 0.25) (layer B.Cu) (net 1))
 (segment (start 182.2489 122.3654) (end 182.2489 121.9) (width 0.25) (layer B.Cu) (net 1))
 (segment (start 183.294 121.8645) (end 182.044 121.861) (width 1.3) (layer F.Cu) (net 1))
 (segment (start 184.544 121.868) (end 183.294 121.8645) (width 1.3) (layer F.Cu) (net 1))
 (segment (start 142.457 110.114) (end 142.011 110.114) (width 0.25) (layer F.Cu) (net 1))
 (segment (start 142.011 110.114) (end 141.871 110.254) (width 0.25) (layer F.Cu) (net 1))
 (segment (start 142.457 110.114) (end 142.014 110.268) (width 1) (layer F.Cu) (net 1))
 (segment (start 142.014 110.268) (end 142.825 110.739) (width 1) (layer F.Cu) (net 1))
 (segment (start 142.9 109.96) (end 142.457 110.114) (width 1) (layer F.Cu) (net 1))
 (segment (start 141.871 110.254) (end 143.041 110.367) (width 1) (layer F.Cu) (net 1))
 (segment (start 147.57 111.635) (end 148.216 111.914) (width 1.3) (layer F.Cu) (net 1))
 (segment (start 143.041 110.367) (end 147.57 111.635) (width 1.86) (layer F.Cu) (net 1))
 (segment (start 149.248 111.952) (end 148.216 111.914) (width 1.3) (layer F.Cu) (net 1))
 (segment (start 182.044 121.861) (end 178.208 120.902) (width 1.86) (layer F.Cu) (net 1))
 (segment (start 178.208 120.902) (end 174.15 119.855) (width 1.86) (layer F.Cu) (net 1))
 (segment (start 174.15 119.855) (end 170.562 118.69) (width 1.86) (layer F.Cu) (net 1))
 (segment (start 170.562 118.69) (end 167.775 117.488) (width 1.86) (layer F.Cu) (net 1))
 (segment (start 167.775 117.488) (end 164.361 115.903) (width 1.86) (layer F.Cu) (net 1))
 (segment (start 164.361 115.903) (end 159.669 114.266) (width 1.86) (layer F.Cu) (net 1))
 (segment (start 159.669 114.266) (end 154.759 113.001) (width 1.86) (layer F.Cu) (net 1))
 (segment (start 154.759 113.001) (end 149.248 111.952) (width 1.86) (layer F.Cu) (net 1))
 (via (at 182.0653 122.549) (size 0.6) (layers F.Cu B.Cu) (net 1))
 (segment (start 173.2009 109.4) (end 173.201 109.4) (width 1) (layer F.Cu) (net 5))
 (segment (start 168.4 109.75) (end 173.2009 109.4) (width 1) (layer F.Cu) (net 5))
 (segment (start 164.746 109.859) (end 168.4 109.75) (width 1) (layer F.Cu) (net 5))
 (segment (start 157.255 109.826) (end 161.346 109.859) (width 1) (layer F.Cu) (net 6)))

